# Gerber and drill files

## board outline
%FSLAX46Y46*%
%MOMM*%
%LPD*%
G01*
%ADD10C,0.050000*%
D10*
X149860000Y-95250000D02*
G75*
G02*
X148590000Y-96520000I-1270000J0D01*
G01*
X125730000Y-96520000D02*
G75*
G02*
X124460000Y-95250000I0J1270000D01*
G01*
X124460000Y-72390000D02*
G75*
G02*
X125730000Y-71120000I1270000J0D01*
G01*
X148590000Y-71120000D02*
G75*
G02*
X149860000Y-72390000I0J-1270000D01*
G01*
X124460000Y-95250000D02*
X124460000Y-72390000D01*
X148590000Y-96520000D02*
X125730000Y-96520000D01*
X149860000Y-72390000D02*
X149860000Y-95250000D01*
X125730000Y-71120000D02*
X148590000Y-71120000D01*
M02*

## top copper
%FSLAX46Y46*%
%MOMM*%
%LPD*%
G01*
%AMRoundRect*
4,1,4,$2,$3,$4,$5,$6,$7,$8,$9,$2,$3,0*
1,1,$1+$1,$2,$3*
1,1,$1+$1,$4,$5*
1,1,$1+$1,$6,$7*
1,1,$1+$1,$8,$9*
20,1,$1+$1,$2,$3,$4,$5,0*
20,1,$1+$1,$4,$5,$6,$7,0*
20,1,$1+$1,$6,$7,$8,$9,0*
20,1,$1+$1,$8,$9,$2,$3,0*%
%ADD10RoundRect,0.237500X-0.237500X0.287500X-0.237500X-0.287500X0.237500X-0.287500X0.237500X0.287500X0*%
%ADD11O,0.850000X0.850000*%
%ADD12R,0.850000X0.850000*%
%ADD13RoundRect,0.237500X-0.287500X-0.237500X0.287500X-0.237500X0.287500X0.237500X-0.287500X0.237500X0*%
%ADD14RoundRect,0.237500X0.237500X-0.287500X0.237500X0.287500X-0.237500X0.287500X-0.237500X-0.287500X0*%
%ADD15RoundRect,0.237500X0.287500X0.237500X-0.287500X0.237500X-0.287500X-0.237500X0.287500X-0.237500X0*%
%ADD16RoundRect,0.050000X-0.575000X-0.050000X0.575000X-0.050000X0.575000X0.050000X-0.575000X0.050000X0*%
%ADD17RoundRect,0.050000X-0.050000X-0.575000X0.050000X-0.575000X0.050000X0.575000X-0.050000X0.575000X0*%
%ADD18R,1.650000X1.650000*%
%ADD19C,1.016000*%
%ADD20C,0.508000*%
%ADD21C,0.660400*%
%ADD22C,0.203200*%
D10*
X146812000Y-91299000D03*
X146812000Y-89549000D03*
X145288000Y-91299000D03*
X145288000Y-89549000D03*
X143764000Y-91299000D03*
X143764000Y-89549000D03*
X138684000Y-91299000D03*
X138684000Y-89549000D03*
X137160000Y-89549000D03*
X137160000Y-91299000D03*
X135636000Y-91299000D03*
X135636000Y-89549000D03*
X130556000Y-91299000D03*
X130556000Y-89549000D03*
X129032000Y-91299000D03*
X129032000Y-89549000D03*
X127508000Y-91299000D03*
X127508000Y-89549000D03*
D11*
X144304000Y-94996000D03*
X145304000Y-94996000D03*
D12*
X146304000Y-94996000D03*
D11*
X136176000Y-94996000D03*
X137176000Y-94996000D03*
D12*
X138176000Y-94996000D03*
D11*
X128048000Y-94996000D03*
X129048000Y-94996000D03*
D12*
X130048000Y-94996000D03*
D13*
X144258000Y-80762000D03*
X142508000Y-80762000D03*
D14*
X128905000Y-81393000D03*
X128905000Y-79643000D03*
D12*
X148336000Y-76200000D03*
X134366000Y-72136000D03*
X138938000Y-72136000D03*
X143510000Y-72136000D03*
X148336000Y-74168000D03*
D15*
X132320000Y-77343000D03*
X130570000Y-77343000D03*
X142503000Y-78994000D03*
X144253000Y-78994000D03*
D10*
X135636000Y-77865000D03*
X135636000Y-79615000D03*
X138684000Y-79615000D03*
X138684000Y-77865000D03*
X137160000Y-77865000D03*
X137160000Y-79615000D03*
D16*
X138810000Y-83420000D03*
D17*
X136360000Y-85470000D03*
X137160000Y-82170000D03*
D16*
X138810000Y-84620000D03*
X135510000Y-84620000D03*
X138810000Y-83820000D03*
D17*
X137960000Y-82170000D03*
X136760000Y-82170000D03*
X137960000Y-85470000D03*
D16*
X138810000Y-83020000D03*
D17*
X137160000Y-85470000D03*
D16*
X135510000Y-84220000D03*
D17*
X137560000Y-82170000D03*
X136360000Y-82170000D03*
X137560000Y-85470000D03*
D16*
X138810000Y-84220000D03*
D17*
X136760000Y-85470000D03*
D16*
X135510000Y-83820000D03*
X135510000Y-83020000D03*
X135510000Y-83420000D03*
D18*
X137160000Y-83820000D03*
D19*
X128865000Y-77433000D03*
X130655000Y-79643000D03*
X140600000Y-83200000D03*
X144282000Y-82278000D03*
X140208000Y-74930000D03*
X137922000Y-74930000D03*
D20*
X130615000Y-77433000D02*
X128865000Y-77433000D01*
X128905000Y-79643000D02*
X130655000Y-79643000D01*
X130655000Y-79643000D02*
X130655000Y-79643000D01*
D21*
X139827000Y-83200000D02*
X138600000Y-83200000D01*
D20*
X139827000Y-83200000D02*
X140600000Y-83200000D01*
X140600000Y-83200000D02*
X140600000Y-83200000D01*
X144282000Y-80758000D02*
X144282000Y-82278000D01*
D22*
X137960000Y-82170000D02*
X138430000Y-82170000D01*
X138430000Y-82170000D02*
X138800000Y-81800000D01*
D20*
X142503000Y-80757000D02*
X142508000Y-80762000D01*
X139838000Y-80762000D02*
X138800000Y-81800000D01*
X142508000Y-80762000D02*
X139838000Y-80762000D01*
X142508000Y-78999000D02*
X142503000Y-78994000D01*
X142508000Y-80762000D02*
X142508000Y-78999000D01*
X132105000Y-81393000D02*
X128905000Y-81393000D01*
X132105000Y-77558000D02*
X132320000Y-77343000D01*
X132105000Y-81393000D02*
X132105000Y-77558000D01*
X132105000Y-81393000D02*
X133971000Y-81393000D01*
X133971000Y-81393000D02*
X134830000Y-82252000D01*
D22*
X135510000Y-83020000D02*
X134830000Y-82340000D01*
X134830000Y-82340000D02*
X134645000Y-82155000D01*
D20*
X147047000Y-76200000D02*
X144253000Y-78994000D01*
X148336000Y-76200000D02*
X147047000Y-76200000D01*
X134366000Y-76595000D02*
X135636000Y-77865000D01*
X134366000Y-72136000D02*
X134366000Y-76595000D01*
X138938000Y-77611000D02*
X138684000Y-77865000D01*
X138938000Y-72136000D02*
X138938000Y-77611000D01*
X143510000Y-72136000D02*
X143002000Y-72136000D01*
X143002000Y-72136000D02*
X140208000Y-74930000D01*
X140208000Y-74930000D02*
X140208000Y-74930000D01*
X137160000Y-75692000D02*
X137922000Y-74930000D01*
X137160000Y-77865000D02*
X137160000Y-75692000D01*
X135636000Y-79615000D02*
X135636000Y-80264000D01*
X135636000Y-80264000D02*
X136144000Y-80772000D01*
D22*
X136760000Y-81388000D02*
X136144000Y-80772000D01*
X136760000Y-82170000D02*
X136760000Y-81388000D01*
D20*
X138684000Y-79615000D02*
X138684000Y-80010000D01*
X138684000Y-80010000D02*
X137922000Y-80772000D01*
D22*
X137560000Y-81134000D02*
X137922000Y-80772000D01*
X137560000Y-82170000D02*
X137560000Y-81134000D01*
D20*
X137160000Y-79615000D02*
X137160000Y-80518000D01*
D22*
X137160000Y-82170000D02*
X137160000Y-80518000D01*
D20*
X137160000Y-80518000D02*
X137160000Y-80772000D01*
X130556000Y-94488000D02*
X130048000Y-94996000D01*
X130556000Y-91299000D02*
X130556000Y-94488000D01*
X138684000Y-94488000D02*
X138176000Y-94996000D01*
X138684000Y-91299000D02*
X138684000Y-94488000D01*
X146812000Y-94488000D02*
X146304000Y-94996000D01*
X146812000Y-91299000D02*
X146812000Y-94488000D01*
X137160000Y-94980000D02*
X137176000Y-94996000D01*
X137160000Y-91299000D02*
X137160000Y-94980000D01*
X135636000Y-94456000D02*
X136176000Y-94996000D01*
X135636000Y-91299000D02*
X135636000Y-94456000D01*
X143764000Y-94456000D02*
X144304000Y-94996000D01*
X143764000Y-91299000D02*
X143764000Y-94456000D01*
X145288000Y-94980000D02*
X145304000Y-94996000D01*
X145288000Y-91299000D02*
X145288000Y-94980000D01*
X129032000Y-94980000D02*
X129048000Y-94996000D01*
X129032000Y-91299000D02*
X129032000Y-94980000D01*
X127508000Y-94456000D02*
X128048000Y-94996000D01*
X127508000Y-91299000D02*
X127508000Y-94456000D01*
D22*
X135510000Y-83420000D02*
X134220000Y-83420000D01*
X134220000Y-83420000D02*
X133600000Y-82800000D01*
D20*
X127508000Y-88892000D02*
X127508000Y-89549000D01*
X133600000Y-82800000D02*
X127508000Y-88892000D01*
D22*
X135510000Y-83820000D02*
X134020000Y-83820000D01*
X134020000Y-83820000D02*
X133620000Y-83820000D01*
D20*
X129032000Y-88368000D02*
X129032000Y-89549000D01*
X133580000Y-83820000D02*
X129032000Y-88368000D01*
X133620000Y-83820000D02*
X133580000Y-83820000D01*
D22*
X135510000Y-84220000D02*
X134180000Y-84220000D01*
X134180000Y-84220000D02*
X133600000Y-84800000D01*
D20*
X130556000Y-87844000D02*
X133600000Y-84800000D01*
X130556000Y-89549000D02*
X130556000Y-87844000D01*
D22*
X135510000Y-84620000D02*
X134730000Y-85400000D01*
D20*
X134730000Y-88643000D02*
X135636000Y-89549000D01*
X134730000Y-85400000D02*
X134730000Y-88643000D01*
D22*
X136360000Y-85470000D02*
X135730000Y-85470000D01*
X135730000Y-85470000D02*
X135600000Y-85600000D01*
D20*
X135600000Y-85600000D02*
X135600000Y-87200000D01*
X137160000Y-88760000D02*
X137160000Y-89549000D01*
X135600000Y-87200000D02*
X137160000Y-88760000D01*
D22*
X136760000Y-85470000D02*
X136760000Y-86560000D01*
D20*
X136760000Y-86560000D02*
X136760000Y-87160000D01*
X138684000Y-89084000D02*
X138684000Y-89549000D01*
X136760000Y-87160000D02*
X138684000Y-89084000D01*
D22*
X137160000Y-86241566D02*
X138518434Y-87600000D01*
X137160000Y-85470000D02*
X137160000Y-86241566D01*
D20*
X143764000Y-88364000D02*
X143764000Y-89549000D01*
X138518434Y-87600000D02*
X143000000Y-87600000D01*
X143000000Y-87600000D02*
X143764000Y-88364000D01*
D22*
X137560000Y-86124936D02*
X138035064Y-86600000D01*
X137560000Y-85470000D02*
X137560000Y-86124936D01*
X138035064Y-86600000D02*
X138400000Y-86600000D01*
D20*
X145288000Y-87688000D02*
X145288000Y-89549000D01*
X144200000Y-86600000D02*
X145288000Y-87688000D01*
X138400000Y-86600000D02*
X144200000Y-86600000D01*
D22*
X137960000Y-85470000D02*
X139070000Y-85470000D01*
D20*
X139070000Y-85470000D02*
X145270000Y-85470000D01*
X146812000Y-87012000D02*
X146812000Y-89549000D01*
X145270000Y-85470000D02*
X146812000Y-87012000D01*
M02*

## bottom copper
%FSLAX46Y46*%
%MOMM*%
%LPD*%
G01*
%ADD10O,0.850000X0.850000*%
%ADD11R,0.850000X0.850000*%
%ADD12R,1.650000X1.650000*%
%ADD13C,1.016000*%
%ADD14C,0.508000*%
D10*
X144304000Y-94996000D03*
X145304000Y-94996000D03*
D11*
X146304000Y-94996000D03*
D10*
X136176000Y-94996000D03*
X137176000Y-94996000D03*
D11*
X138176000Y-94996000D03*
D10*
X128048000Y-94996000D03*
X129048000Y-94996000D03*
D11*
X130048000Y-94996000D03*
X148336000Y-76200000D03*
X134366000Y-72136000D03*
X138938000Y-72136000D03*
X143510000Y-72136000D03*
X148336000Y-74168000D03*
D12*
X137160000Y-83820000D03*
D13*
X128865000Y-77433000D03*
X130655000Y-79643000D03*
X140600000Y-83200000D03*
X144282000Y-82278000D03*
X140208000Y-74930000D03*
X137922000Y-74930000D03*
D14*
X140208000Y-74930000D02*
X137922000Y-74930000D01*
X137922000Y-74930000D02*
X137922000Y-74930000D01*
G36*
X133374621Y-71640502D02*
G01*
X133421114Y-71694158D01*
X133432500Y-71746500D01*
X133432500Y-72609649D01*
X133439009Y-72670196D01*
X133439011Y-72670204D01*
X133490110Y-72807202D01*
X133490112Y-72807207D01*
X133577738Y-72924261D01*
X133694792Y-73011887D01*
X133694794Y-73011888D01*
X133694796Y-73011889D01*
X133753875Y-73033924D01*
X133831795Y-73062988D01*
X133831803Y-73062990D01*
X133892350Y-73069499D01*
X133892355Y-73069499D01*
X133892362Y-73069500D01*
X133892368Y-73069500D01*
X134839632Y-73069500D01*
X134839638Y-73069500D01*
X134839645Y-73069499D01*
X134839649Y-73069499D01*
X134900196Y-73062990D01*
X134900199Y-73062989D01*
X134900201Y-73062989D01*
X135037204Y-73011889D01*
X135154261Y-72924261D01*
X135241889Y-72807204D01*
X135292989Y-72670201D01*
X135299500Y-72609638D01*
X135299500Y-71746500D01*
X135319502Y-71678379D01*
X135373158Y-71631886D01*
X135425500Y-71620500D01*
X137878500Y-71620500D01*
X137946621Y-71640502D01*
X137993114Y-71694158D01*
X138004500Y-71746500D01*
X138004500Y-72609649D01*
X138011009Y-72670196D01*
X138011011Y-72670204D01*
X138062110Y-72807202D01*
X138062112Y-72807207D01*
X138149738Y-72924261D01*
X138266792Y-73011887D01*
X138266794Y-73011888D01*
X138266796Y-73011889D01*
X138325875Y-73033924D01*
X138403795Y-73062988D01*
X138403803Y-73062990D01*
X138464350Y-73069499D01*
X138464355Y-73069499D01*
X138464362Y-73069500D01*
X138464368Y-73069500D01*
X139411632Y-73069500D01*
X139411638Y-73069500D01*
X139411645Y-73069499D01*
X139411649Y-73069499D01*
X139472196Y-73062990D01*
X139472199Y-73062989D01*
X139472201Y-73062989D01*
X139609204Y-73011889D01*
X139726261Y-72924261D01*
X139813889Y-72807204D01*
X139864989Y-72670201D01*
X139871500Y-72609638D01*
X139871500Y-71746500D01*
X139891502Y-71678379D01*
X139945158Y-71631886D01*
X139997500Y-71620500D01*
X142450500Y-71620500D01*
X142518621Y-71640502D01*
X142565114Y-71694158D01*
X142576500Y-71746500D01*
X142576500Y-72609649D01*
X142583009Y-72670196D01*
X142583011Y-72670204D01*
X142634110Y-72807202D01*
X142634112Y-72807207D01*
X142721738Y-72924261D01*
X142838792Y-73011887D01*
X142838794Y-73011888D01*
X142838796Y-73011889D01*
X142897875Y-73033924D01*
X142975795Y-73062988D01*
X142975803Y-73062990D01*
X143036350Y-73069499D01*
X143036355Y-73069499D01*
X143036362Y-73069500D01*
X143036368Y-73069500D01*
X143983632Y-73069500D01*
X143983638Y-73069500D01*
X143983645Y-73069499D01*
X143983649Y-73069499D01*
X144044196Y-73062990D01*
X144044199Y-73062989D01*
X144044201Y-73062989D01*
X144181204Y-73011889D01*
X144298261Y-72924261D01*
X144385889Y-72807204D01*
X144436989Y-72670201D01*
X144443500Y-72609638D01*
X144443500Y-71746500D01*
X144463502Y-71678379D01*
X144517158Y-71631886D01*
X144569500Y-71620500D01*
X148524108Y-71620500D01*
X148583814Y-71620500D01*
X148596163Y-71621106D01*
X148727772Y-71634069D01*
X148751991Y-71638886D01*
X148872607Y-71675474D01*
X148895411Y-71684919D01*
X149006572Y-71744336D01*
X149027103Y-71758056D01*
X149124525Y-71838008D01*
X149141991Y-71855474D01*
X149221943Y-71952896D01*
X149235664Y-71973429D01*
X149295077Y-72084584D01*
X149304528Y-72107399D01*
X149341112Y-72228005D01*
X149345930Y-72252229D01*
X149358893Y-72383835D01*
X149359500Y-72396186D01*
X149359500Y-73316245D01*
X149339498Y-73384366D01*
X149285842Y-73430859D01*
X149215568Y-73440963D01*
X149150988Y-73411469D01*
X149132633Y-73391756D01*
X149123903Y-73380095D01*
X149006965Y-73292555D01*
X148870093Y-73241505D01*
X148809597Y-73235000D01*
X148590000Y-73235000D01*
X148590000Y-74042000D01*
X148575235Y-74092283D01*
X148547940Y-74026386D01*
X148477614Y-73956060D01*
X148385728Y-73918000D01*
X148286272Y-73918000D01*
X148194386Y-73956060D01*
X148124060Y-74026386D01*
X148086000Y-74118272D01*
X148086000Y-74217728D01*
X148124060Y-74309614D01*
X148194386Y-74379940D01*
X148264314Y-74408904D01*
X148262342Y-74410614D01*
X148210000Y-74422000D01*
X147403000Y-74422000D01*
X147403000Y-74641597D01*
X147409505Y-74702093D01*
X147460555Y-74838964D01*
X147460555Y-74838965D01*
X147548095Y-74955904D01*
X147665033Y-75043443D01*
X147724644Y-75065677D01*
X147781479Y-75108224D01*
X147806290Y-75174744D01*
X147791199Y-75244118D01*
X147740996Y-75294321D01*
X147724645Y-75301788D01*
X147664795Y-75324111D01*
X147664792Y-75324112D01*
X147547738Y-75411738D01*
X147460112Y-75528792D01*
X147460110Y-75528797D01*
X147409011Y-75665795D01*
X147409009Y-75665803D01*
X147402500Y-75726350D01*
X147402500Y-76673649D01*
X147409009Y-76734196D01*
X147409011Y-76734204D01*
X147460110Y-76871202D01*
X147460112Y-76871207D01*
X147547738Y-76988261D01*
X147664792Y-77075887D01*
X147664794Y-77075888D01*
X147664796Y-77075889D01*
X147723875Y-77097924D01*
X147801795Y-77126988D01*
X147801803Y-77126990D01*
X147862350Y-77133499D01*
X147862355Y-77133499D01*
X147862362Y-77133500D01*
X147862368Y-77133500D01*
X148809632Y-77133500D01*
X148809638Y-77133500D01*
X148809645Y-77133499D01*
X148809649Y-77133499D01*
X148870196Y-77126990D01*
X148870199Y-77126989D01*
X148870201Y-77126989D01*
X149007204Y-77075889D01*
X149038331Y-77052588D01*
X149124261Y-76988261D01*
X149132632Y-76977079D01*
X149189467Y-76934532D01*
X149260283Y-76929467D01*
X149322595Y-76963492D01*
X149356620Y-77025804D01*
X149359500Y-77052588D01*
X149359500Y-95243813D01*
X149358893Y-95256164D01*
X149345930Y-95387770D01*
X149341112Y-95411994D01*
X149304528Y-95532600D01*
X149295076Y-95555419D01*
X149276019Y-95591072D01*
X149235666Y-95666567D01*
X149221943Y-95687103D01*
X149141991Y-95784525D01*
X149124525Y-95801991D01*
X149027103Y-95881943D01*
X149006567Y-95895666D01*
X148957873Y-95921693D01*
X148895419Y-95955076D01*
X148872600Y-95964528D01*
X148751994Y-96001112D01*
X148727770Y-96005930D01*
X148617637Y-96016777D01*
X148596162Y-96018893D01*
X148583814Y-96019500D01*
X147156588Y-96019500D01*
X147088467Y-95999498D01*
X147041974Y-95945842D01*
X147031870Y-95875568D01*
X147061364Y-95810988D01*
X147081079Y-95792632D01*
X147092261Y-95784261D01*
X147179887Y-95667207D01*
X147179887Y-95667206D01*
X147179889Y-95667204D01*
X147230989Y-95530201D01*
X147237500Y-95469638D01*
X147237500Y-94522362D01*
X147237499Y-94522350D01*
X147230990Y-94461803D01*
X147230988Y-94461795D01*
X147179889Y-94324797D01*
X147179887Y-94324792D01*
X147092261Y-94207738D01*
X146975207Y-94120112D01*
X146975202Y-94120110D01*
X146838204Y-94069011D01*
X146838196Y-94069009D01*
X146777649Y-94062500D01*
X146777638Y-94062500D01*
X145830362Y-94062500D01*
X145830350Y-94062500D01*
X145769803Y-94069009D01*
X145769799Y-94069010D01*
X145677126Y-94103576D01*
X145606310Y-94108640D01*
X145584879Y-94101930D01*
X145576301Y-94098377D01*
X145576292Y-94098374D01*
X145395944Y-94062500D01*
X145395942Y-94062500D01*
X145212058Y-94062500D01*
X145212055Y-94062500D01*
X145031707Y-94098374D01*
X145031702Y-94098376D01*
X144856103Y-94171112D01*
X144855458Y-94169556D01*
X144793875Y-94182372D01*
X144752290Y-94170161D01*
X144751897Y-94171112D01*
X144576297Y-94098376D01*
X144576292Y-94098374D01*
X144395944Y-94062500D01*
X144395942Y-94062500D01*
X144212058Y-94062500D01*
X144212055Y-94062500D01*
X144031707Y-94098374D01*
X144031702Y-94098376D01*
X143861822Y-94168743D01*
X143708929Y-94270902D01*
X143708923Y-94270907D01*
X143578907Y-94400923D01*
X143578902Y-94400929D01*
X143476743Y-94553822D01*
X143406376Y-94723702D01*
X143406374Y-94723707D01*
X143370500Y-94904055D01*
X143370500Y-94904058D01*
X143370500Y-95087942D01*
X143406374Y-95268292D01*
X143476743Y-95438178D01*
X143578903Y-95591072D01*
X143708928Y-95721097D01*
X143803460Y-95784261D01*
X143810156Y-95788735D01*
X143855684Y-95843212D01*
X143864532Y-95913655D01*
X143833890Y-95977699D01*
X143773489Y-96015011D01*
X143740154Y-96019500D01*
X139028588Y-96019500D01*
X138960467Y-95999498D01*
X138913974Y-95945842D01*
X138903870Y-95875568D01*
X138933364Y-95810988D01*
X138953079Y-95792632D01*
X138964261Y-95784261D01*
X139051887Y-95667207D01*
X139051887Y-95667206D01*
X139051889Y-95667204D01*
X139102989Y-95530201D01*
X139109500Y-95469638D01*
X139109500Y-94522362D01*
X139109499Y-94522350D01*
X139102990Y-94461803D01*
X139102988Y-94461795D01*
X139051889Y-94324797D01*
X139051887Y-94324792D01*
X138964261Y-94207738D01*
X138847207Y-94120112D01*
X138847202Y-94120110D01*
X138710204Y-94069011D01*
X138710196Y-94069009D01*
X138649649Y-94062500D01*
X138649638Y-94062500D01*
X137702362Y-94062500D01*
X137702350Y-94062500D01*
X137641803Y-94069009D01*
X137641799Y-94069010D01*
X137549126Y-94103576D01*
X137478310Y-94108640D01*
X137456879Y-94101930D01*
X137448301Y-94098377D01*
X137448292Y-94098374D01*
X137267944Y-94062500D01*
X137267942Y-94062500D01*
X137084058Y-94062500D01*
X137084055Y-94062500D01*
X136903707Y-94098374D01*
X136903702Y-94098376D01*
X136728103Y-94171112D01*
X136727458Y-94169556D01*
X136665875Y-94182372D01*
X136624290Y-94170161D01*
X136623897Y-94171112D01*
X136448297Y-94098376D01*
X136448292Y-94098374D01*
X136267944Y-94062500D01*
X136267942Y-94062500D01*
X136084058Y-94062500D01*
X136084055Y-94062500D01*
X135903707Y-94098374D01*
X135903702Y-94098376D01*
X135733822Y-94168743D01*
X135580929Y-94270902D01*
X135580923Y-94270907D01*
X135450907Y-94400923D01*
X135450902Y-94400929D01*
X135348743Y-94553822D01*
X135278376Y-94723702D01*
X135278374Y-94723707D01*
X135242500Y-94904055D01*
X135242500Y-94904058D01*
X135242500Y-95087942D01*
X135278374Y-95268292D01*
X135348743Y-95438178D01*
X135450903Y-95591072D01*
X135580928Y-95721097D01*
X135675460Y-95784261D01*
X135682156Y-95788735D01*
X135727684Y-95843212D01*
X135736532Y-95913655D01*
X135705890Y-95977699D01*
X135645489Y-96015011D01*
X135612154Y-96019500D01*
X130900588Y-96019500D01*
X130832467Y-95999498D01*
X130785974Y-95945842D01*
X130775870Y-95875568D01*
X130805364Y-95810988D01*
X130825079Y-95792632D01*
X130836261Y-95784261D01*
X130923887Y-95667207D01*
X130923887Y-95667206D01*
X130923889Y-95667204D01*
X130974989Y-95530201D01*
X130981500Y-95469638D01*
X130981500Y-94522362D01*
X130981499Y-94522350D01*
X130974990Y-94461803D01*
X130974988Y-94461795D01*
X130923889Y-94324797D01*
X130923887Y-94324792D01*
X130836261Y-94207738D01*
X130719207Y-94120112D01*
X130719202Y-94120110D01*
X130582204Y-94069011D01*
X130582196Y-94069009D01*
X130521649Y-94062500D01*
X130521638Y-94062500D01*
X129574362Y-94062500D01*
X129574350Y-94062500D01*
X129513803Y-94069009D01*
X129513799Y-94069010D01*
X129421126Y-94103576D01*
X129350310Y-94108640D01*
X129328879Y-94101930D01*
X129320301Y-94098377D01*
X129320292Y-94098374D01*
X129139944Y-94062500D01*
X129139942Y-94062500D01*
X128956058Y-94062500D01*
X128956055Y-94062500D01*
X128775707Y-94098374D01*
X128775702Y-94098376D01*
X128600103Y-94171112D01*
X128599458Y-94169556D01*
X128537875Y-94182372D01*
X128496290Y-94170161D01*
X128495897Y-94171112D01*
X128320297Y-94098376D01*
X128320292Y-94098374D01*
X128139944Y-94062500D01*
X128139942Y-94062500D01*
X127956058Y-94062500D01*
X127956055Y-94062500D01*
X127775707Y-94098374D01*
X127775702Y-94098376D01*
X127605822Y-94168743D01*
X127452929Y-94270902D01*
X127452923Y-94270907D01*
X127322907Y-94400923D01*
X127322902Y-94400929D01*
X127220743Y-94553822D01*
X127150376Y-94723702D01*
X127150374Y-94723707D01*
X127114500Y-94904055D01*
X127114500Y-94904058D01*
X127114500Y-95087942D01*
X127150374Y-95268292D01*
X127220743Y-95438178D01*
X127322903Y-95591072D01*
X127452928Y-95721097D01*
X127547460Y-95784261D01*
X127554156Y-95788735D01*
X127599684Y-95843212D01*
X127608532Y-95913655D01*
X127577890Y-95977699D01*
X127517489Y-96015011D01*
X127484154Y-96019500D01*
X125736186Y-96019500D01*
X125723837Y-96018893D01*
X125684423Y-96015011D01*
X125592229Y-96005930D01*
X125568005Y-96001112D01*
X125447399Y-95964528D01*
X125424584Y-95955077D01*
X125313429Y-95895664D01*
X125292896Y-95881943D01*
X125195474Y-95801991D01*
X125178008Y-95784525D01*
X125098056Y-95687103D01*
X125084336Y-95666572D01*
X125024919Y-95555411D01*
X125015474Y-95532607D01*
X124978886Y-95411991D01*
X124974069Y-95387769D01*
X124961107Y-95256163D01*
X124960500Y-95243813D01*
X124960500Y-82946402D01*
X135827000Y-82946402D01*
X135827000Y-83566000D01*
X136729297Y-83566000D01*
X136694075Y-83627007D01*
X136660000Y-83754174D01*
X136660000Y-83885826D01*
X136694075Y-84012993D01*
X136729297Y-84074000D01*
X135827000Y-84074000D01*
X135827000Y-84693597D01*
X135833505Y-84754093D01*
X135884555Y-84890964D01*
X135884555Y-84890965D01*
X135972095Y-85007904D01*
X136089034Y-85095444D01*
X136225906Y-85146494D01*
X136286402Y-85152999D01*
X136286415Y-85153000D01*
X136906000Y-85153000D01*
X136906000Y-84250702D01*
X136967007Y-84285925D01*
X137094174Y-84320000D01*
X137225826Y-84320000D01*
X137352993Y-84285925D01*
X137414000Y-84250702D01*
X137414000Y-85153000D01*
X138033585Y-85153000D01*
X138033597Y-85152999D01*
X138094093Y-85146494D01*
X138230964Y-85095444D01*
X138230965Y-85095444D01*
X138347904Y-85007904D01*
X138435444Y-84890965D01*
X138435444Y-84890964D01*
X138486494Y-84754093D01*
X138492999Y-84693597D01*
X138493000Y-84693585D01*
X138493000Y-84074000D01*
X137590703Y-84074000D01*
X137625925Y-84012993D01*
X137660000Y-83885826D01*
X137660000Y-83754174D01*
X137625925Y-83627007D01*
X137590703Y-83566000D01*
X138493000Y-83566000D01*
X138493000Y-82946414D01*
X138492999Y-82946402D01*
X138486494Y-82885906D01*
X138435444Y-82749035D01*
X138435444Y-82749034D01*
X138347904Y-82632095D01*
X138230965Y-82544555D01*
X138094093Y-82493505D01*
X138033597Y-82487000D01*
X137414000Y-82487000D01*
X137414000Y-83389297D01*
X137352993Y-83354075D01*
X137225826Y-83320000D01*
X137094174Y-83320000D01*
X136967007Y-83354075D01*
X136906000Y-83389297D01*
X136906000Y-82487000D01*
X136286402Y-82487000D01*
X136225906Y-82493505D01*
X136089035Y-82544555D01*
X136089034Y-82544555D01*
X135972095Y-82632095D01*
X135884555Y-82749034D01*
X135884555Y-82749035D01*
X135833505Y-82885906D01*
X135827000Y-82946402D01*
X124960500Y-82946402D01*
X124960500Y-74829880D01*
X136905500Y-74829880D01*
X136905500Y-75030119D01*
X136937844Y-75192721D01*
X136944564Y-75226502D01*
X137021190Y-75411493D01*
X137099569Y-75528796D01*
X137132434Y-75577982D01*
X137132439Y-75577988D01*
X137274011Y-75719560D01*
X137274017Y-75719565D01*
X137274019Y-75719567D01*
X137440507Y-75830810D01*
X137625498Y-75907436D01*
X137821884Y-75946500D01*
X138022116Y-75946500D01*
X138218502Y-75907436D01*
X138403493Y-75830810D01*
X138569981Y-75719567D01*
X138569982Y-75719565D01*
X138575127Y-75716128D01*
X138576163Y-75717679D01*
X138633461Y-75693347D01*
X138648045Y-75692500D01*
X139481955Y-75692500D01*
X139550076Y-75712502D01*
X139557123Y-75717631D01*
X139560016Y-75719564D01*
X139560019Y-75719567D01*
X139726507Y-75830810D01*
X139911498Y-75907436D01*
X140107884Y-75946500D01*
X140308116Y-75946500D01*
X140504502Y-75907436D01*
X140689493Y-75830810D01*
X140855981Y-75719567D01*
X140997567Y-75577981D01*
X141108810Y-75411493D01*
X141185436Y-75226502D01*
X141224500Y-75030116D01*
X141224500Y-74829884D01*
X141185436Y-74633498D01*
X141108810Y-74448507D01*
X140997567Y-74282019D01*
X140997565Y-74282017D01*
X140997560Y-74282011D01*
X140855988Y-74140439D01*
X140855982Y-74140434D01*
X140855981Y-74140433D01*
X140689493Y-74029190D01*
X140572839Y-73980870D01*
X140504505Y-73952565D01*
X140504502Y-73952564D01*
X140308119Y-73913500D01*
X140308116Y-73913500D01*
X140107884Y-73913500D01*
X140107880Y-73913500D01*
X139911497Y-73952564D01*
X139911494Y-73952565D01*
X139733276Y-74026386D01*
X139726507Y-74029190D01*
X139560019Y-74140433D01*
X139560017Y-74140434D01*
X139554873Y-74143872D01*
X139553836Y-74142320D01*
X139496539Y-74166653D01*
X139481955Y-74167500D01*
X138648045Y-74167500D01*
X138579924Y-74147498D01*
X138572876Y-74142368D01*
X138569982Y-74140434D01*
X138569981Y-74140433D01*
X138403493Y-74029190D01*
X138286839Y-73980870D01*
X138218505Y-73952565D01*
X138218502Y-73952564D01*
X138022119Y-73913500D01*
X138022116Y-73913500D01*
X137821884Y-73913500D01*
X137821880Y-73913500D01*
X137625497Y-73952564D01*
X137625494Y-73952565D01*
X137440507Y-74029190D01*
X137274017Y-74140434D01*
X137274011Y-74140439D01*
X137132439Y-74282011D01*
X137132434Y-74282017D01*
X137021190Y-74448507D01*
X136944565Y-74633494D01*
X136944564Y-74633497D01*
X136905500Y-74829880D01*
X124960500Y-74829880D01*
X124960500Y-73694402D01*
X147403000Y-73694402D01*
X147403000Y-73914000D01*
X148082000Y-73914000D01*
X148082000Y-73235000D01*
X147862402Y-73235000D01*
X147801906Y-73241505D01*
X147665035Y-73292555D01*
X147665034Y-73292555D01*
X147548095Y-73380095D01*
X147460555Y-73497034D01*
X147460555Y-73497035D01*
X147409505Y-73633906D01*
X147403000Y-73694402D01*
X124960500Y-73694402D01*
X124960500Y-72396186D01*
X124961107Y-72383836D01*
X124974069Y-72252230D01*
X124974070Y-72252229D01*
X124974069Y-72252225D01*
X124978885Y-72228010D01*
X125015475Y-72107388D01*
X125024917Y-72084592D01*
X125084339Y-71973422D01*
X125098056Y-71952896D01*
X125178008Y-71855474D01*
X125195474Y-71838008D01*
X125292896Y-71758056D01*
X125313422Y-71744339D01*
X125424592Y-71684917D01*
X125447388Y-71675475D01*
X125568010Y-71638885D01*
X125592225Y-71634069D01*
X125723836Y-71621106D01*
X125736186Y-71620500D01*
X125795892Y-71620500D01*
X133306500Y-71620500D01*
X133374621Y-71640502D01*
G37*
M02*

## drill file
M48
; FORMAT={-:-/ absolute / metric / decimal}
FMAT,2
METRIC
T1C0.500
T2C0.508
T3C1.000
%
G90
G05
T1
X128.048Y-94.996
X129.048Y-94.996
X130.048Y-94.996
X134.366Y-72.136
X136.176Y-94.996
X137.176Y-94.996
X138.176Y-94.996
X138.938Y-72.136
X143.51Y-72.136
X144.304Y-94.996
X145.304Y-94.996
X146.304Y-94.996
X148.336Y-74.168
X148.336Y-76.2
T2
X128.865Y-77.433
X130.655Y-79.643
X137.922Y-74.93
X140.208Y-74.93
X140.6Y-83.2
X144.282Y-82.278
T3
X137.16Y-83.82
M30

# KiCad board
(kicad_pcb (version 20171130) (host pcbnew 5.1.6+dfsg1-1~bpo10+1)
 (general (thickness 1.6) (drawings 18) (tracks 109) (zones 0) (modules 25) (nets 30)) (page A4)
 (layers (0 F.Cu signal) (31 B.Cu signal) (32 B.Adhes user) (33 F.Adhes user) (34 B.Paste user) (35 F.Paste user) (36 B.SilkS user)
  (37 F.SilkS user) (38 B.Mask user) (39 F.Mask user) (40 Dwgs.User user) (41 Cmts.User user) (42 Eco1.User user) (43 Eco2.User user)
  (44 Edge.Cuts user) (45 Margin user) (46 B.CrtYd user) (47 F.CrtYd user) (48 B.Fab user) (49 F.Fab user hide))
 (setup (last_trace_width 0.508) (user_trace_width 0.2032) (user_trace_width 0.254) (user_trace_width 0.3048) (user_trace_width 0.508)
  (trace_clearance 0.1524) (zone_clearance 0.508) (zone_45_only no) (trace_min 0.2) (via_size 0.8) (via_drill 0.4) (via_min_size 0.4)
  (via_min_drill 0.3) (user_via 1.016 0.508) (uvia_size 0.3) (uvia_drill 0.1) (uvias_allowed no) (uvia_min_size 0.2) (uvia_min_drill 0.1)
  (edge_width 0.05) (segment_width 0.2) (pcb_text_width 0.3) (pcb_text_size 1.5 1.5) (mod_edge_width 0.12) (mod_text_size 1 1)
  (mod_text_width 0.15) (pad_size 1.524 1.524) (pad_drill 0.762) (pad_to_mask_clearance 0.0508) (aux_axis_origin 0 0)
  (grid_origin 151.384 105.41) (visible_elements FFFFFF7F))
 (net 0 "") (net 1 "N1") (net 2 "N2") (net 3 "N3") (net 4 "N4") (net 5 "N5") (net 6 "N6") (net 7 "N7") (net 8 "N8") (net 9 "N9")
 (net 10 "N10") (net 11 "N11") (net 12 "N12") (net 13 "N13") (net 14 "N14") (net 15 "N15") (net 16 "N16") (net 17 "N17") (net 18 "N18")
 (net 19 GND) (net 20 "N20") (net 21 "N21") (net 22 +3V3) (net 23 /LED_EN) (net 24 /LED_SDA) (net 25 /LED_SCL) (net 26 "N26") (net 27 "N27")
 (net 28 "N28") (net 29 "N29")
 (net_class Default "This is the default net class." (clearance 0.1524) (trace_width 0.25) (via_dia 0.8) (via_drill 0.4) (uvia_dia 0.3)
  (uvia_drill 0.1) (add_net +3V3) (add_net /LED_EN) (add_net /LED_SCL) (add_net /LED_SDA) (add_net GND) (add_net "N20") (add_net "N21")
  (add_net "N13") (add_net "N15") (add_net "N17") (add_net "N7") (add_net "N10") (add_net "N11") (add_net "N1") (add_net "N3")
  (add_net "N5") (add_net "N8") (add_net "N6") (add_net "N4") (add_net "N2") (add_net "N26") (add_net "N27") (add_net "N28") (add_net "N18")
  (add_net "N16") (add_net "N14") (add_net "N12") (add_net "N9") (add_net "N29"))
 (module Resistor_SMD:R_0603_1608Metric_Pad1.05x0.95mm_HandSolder (layer F.Cu) (at 146.812 90.424 270)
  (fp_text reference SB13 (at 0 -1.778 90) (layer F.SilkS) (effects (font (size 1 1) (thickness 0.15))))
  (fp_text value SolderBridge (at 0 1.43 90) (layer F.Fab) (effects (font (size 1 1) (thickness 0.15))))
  (pad 2 smd roundrect (at 0.875 0 270) (size 1.05 0.95) (layers F.Cu F.Paste F.Mask) (roundrect_rratio 0.25) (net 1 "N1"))
  (pad 1 smd roundrect (at -0.875 0 270) (size 1.05 0.95) (layers F.Cu F.Paste F.Mask) (roundrect_rratio 0.25) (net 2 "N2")))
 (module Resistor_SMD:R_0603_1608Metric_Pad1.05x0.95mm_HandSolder (layer F.Cu) (at 145.288 90.424 270)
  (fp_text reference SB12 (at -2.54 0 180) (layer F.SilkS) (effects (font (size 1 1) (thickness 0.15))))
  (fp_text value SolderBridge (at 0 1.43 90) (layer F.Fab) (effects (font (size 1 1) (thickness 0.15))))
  (pad 2 smd roundrect (at 0.875 0 270) (size 1.05 0.95) (layers F.Cu F.Paste F.Mask) (roundrect_rratio 0.25) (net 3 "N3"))
  (pad 1 smd roundrect (at -0.875 0 270) (size 1.05 0.95) (layers F.Cu F.Paste F.Mask) (roundrect_rratio 0.25) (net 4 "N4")))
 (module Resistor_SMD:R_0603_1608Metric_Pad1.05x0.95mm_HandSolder (layer F.Cu) (at 143.764 90.424 270)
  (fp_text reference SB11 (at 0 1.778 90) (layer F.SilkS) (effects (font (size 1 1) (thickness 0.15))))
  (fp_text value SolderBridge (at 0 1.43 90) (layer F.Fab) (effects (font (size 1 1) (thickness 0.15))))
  (pad 2 smd roundrect (at 0.875 0 270) (size 1.05 0.95) (layers F.Cu F.Paste F.Mask) (roundrect_rratio 0.25) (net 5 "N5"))
  (pad 1 smd roundrect (at -0.875 0 270) (size 1.05 0.95) (layers F.Cu F.Paste F.Mask) (roundrect_rratio 0.25) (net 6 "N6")))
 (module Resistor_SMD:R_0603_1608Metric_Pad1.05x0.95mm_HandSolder (layer F.Cu) (at 138.684 90.424 270)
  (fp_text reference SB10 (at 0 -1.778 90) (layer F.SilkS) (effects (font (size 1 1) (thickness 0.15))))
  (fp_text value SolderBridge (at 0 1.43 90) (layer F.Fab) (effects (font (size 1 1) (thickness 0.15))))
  (pad 2 smd roundrect (at 0.875 0 270) (size 1.05 0.95) (layers F.Cu F.Paste F.Mask) (roundrect_rratio 0.25) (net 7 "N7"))
  (pad 1 smd roundrect (at -0.875 0 270) (size 1.05 0.95) (layers F.Cu F.Paste F.Mask) (roundrect_rratio 0.25) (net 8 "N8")))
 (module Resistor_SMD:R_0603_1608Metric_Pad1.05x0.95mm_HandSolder (layer F.Cu) (at 137.16 90.424 270)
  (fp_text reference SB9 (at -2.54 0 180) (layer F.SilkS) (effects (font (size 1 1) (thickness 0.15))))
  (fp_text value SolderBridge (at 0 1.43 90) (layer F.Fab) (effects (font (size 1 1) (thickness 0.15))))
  (pad 1 smd roundrect (at -0.875 0 270) (size 1.05 0.95) (layers F.Cu F.Paste F.Mask) (roundrect_rratio 0.25) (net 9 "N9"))
  (pad 2 smd roundrect (at 0.875 0 270) (size 1.05 0.95) (layers F.Cu F.Paste F.Mask) (roundrect_rratio 0.25) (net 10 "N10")))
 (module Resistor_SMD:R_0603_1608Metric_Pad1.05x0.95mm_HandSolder (layer F.Cu) (at 135.636 90.424 270)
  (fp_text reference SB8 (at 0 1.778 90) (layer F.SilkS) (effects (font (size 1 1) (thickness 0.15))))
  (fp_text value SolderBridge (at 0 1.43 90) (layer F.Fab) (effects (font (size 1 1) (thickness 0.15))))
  (pad 2 smd roundrect (at 0.875 0 270) (size 1.05 0.95) (layers F.Cu F.Paste F.Mask) (roundrect_rratio 0.25) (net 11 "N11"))
  (pad 1 smd roundrect (at -0.875 0 270) (size 1.05 0.95) (layers F.Cu F.Paste F.Mask) (roundrect_rratio 0.25) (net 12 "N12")))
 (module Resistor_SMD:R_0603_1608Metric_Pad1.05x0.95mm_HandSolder (layer F.Cu) (at 130.556 90.424 270)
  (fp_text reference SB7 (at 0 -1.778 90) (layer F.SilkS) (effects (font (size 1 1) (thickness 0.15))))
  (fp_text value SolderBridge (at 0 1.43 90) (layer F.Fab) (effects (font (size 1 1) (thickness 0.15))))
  (pad 2 smd roundrect (at 0.875 0 270) (size 1.05 0.95) (layers F.Cu F.Paste F.Mask) (roundrect_rratio 0.25) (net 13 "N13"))
  (pad 1 smd roundrect (at -0.875 0 270) (size 1.05 0.95) (layers F.Cu F.Paste F.Mask) (roundrect_rratio 0.25) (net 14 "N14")))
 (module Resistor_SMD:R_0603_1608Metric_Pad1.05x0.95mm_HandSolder (layer F.Cu) (at 129.032 90.424 270)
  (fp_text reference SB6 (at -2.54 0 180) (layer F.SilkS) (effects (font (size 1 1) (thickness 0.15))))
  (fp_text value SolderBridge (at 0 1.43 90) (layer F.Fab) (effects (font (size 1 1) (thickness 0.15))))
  (pad 2 smd roundrect (at 0.875 0 270) (size 1.05 0.95) (layers F.Cu F.Paste F.Mask) (roundrect_rratio 0.25) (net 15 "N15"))
  (pad 1 smd roundrect (at -0.875 0 270) (size 1.05 0.95) (layers F.Cu F.Paste F.Mask) (roundrect_rratio 0.25) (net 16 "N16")))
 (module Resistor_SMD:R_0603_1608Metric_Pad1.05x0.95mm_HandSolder (layer F.Cu) (at 127.508 90.424 270)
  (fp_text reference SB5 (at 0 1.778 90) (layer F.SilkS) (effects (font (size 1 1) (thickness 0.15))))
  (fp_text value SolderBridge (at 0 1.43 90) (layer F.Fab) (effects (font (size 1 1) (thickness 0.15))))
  (pad 2 smd roundrect (at 0.875 0 270) (size 1.05 0.95) (layers F.Cu F.Paste F.Mask) (roundrect_rratio 0.25) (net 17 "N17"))
  (pad 1 smd roundrect (at -0.875 0 270) (size 1.05 0.95) (layers F.Cu F.Paste F.Mask) (roundrect_rratio 0.25) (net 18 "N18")))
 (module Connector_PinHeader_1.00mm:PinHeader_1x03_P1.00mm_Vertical (layer F.Cu) (at 146.304 94.996 270)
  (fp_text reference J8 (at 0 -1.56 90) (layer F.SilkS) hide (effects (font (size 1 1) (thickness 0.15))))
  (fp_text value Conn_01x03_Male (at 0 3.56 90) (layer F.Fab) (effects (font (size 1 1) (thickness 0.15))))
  (pad 3 thru_hole oval (at 0 2 270) (size 0.85 0.85) (drill 0.5) (layers *.Cu *.Mask) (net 5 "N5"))
  (pad 2 thru_hole oval (at 0 1 270) (size 0.85 0.85) (drill 0.5) (layers *.Cu *.Mask) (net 3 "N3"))
  (pad 1 thru_hole rect (at 0 0 270) (size 0.85 0.85) (drill 0.5) (layers *.Cu *.Mask) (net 1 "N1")))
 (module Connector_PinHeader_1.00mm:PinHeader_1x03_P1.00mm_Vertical (layer F.Cu) (at 138.176 94.996 270)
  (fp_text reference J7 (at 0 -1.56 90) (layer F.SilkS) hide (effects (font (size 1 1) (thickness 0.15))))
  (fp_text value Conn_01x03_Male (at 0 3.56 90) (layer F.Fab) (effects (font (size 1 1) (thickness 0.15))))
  (pad 3 thru_hole oval (at 0 2 270) (size 0.85 0.85) (drill 0.5) (layers *.Cu *.Mask) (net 11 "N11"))
  (pad 2 thru_hole oval (at 0 1 270) (size 0.85 0.85) (drill 0.5) (layers *.Cu *.Mask) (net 10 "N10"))
  (pad 1 thru_hole rect (at 0 0 270) (size 0.85 0.85) (drill 0.5) (layers *.Cu *.Mask) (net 7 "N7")))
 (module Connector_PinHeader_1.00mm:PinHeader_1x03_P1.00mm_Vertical (layer F.Cu) (at 130.048 94.996 270)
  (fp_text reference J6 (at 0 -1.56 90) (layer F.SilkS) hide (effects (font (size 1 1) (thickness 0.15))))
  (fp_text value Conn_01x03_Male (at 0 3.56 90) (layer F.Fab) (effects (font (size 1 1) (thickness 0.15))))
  (pad 3 thru_hole oval (at 0 2 270) (size 0.85 0.85) (drill 0.5) (layers *.Cu *.Mask) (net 17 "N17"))
  (pad 2 thru_hole oval (at 0 1 270) (size 0.85 0.85) (drill 0.5) (layers *.Cu *.Mask) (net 15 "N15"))
  (pad 1 thru_hole rect (at 0 0 270) (size 0.85 0.85) (drill 0.5) (layers *.Cu *.Mask) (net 13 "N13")))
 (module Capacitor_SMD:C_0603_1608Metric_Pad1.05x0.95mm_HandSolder (layer F.Cu) (at 143.383 80.762)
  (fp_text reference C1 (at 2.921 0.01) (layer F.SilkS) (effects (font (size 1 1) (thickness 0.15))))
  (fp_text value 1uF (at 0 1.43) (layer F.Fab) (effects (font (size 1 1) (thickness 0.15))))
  (pad 2 smd roundrect (at 0.875 0) (size 1.05 0.95) (layers F.Cu F.Paste F.Mask) (roundrect_rratio 0.25) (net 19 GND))
  (pad 1 smd roundrect (at -0.875 0) (size 1.05 0.95) (layers F.Cu F.Paste F.Mask) (roundrect_rratio 0.25) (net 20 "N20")))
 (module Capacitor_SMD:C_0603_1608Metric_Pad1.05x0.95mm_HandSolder (layer F.Cu) (at 128.905 80.518 90)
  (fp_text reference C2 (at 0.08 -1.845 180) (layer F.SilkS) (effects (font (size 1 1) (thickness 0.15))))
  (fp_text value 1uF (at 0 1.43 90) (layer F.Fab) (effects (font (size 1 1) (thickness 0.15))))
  (pad 1 smd roundrect (at -0.875 0 90) (size 1.05 0.95) (layers F.Cu F.Paste F.Mask) (roundrect_rratio 0.25) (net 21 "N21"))
  (pad 2 smd roundrect (at 0.875 0 90) (size 1.05 0.95) (layers F.Cu F.Paste F.Mask) (roundrect_rratio 0.25) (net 19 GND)))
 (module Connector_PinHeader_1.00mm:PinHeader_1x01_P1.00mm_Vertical (layer F.Cu) (at 148.336 76.2)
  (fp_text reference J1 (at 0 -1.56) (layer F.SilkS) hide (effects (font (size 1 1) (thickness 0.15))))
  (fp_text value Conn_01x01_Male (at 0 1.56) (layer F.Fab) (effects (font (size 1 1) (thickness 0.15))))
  (pad 1 thru_hole rect (at 0 0) (size 0.85 0.85) (drill 0.5) (layers *.Cu *.Mask) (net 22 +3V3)))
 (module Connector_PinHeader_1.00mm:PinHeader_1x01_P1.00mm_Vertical (layer F.Cu) (at 134.366 72.136)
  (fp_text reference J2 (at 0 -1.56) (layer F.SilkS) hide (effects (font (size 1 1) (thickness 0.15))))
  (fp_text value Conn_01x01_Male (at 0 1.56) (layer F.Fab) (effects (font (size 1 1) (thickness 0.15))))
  (pad 1 thru_hole rect (at 0 0) (size 0.85 0.85) (drill 0.5) (layers *.Cu *.Mask) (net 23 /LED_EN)))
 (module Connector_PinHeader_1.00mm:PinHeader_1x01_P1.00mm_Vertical (layer F.Cu) (at 138.938 72.136)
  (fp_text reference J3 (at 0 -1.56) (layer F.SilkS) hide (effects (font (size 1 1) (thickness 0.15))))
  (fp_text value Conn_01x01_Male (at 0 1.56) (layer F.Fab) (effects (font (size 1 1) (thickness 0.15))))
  (pad 1 thru_hole rect (at 0 0) (size 0.85 0.85) (drill 0.5) (layers *.Cu *.Mask) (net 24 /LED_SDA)))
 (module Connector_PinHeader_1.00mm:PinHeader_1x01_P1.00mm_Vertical (layer F.Cu) (at 143.51 72.136)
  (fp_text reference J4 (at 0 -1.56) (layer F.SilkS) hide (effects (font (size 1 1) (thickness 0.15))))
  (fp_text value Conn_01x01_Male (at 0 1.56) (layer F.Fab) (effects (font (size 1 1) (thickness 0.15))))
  (pad 1 thru_hole rect (at 0 0) (size 0.85 0.85) (drill 0.5) (layers *.Cu *.Mask) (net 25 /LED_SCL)))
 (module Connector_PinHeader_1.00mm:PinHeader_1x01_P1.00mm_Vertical (layer F.Cu) (at 148.336 74.168)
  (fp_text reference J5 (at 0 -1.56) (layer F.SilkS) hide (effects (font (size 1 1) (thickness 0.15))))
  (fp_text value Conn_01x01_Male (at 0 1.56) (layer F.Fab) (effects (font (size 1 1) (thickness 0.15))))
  (pad 1 thru_hole rect (at 0 0) (size 0.85 0.85) (drill 0.5) (layers *.Cu *.Mask) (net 19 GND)))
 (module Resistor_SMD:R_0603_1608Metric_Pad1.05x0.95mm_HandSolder (layer F.Cu) (at 131.445 77.343 180)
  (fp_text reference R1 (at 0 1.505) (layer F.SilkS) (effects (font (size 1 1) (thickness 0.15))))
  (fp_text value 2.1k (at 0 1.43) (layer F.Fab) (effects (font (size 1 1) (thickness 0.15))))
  (pad 1 smd roundrect (at -0.875 0 180) (size 1.05 0.95) (layers F.Cu F.Paste F.Mask) (roundrect_rratio 0.25) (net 21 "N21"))
  (pad 2 smd roundrect (at 0.875 0 180) (size 1.05 0.95) (layers F.Cu F.Paste F.Mask) (roundrect_rratio 0.25) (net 19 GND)))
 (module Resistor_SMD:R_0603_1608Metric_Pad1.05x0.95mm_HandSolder (layer F.Cu) (at 143.378 78.994 180)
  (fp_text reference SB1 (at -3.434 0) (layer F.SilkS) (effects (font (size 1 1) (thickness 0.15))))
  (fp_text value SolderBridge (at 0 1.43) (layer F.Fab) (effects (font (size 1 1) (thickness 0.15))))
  (pad 2 smd roundrect (at 0.875 0 180) (size 1.05 0.95) (layers F.Cu F.Paste F.Mask) (roundrect_rratio 0.25) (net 20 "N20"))
  (pad 1 smd roundrect (at -0.875 0 180) (size 1.05 0.95) (layers F.Cu F.Paste F.Mask) (roundrect_rratio 0.25) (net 22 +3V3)))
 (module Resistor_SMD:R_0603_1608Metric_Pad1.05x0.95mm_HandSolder (layer F.Cu) (at 135.636 78.74 270)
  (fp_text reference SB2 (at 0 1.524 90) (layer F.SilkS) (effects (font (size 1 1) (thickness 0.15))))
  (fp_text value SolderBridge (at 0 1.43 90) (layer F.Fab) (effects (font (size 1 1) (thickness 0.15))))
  (pad 1 smd roundrect (at -0.875 0 270) (size 1.05 0.95) (layers F.Cu F.Paste F.Mask) (roundrect_rratio 0.25) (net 23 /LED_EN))
  (pad 2 smd roundrect (at 0.875 0 270) (size 1.05 0.95) (layers F.Cu F.Paste F.Mask) (roundrect_rratio 0.25) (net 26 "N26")))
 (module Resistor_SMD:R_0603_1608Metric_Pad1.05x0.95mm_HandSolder (layer F.Cu) (at 138.684 78.74 270)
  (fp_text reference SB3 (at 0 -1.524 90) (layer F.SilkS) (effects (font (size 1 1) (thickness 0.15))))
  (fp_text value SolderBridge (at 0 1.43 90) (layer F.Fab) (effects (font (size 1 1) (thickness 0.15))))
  (pad 2 smd roundrect (at 0.875 0 270) (size 1.05 0.95) (layers F.Cu F.Paste F.Mask) (roundrect_rratio 0.25) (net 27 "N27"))
  (pad 1 smd roundrect (at -0.875 0 270) (size 1.05 0.95) (layers F.Cu F.Paste F.Mask) (roundrect_rratio 0.25) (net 24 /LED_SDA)))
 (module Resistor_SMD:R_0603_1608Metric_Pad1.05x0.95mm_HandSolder (layer F.Cu) (at 137.16 78.74 270)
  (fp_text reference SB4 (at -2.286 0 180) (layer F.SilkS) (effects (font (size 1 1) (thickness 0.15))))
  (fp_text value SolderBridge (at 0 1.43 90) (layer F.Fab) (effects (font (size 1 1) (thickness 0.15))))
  (pad 1 smd roundrect (at -0.875 0 270) (size 1.05 0.95) (layers F.Cu F.Paste F.Mask) (roundrect_rratio 0.25) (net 25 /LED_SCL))
  (pad 2 smd roundrect (at 0.875 0 270) (size 1.05 0.95) (layers F.Cu F.Paste F.Mask) (roundrect_rratio 0.25) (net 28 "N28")))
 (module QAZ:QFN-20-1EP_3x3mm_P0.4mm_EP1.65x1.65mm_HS (layer F.Cu) (at 137.16 83.82)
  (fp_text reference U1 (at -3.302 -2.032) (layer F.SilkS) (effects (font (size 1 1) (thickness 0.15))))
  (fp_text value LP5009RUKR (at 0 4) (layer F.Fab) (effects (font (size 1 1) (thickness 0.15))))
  (pad 14 smd roundrect (at 1.65 -0.4) (size 1.25 0.2) (layers F.Cu F.Paste F.Mask) (roundrect_rratio 0.25) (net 19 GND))
  (pad 6 smd roundrect (at -0.8 1.65) (size 0.2 1.25) (layers F.Cu F.Paste F.Mask) (roundrect_rratio 0.25) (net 9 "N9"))
  (pad 18 smd roundrect (at 0 -1.65) (size 0.2 1.25) (layers F.Cu F.Paste F.Mask) (roundrect_rratio 0.25) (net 28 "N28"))
  (pad 11 smd roundrect (at 1.65 0.8) (size 1.25 0.2) (layers F.Cu F.Paste F.Mask) (roundrect_rratio 0.25))
  (pad 5 smd roundrect (at -1.65 0.8) (size 1.25 0.2) (layers F.Cu F.Paste F.Mask) (roundrect_rratio 0.25) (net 12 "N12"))
  (pad 13 smd roundrect (at 1.65 0) (size 1.25 0.2) (layers F.Cu F.Paste F.Mask) (roundrect_rratio 0.25))
  (pad 16 smd roundrect (at 0.8 -1.65) (size 0.2 1.25) (layers F.Cu F.Paste F.Mask) (roundrect_rratio 0.25) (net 20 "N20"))
  (pad 19 smd roundrect (at -0.4 -1.65) (size 0.2 1.25) (layers F.Cu F.Paste F.Mask) (roundrect_rratio 0.25) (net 26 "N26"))
  (pad 10 smd roundrect (at 0.8 1.65) (size 0.2 1.25) (layers F.Cu F.Paste F.Mask) (roundrect_rratio 0.25) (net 2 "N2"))
  (pad 15 smd roundrect (at 1.65 -0.8) (size 1.25 0.2) (layers F.Cu F.Paste F.Mask) (roundrect_rratio 0.25) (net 19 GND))
  (pad 8 smd roundrect (at 0 1.65) (size 0.2 1.25) (layers F.Cu F.Paste F.Mask) (roundrect_rratio 0.25) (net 6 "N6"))
  (pad 4 smd roundrect (at -1.65 0.4) (size 1.25 0.2) (layers F.Cu F.Paste F.Mask) (roundrect_rratio 0.25) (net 14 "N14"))
  (pad 17 smd roundrect (at 0.4 -1.65) (size 0.2 1.25) (layers F.Cu F.Paste F.Mask) (roundrect_rratio 0.25) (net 27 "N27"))
  (pad 20 smd roundrect (at -0.8 -1.65) (size 0.2 1.25) (layers F.Cu F.Paste F.Mask) (roundrect_rratio 0.25) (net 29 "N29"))
  (pad 9 smd roundrect (at 0.4 1.65) (size 0.2 1.25) (layers F.Cu F.Paste F.Mask) (roundrect_rratio 0.25) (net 4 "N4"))
  (pad 12 smd roundrect (at 1.65 0.4) (size 1.25 0.2) (layers F.Cu F.Paste F.Mask) (roundrect_rratio 0.25))
  (pad 7 smd roundrect (at -0.4 1.65) (size 0.2 1.25) (layers F.Cu F.Paste F.Mask) (roundrect_rratio 0.25) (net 8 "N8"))
  (pad 3 smd roundrect (at -1.65 0) (size 1.25 0.2) (layers F.Cu F.Paste F.Mask) (roundrect_rratio 0.25) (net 16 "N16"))
  (pad 1 smd roundrect (at -1.65 -0.8) (size 1.25 0.2) (layers F.Cu F.Paste F.Mask) (roundrect_rratio 0.25) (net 21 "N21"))
  (pad 2 smd roundrect (at -1.65 -0.4) (size 1.25 0.2) (layers F.Cu F.Paste F.Mask) (roundrect_rratio 0.25) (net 18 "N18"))
  (pad 21 thru_hole rect (at 0 0) (size 1.65 1.65) (drill 1) (layers *.Cu *.Mask) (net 19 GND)))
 (gr_arc (start 148.59 95.25) (end 148.59 96.52) (angle -90) (layer Edge.Cuts) (width 0.05))
 (gr_arc (start 125.73 95.25) (end 124.46 95.25) (angle -90) (layer Edge.Cuts) (width 0.05))
 (gr_arc (start 125.73 72.39) (end 125.73 71.12) (angle -90) (layer Edge.Cuts) (width 0.05))
 (gr_arc (start 148.59 72.39) (end 149.86 72.39) (angle -90) (layer Edge.Cuts) (width 0.05))
 (gr_line (start 124.46 95.25) (end 124.46 72.39) (layer Edge.Cuts) (width 0.05))
 (gr_line (start 148.59 96.52) (end 125.73 96.52) (layer Edge.Cuts) (width 0.05))
 (gr_line (start 149.86 72.39) (end 149.86 95.25) (layer Edge.Cuts) (width 0.05))
 (gr_line (start 125.73 71.12) (end 148.59 71.12) (layer Edge.Cuts) (width 0.05))
 (via (at 128.865 77.433) (size 1.016) (drill 0.508) (layers F.Cu B.Cu) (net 19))
 (segment (start 130.615 77.433) (end 128.865 77.433) (width 0.508) (layer F.Cu) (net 19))
 (segment (start 128.905 79.643) (end 130.655 79.643) (width 0.508) (layer F.Cu) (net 19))
 (segment (start 130.655 79.643) (end 130.655 79.643) (width 0.508) (layer F.Cu) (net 19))
 (via (at 130.655 79.643) (size 1.016) (drill 0.508) (layers F.Cu B.Cu) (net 19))
 (segment (start 139.827 83.2) (end 138.6 83.2) (width 0.6604) (layer F.Cu) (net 19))
 (segment (start 139.827 83.2) (end 140.6 83.2) (width 0.508) (layer F.Cu) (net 19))
 (segment (start 140.6 83.2) (end 140.6 83.2) (width 0.508) (layer F.Cu) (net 19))
 (via (at 140.6 83.2) (size 1.016) (drill 0.508) (layers F.Cu B.Cu) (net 19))
 (segment (start 144.282 80.758) (end 144.282 82.278) (width 0.508) (layer F.Cu) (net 19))
 (via (at 144.282 82.278) (size 1.016) (drill 0.508) (layers F.Cu B.Cu) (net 19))
 (segment (start 137.96 82.17) (end 138.43 82.17) (width 0.2032) (layer F.Cu) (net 20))
 (segment (start 138.43 82.17) (end 138.8 81.8) (width 0.2032) (layer F.Cu) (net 20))
 (segment (start 142.503 80.757) (end 142.508 80.762) (width 0.508) (layer F.Cu) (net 20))
 (segment (start 139.838 80.762) (end 138.8 81.8) (width 0.508) (layer F.Cu) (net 20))
 (segment (start 142.508 80.762) (end 139.838 80.762) (width 0.508) (layer F.Cu) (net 20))
 (segment (start 142.508 78.999) (end 142.503 78.994) (width 0.508) (layer F.Cu) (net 20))
 (segment (start 142.508 80.762) (end 142.508 78.999) (width 0.508) (layer F.Cu) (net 20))
 (segment (start 132.105 81.393) (end 128.905 81.393) (width 0.508) (layer F.Cu) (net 21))
 (segment (start 132.105 77.558) (end 132.32 77.343) (width 0.508) (layer F.Cu) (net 21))
 (segment (start 132.105 81.393) (end 132.105 77.558) (width 0.508) (layer F.Cu) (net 21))
 (segment (start 132.105 81.393) (end 133.971 81.393) (width 0.508) (layer F.Cu) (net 21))
 (segment (start 133.971 81.393) (end 134.83 82.252) (width 0.508) (layer F.Cu) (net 21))
 (segment (start 135.51 83.02) (end 134.83 82.34) (width 0.2032) (layer F.Cu) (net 21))
 (segment (start 134.83 82.34) (end 134.645 82.155) (width 0.2032) (layer F.Cu) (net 21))
 (segment (start 147.047 76.2) (end 144.253 78.994) (width 0.508) (layer F.Cu) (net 22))
 (segment (start 148.336 76.2) (end 147.047 76.2) (width 0.508) (layer F.Cu) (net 22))
 (segment (start 134.366 76.595) (end 135.636 77.865) (width 0.508) (layer F.Cu) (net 23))
 (segment (start 134.366 72.136) (end 134.366 76.595) (width 0.508) (layer F.Cu) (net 23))
 (segment (start 138.938 77.611) (end 138.684 77.865) (width 0.508) (layer F.Cu) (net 24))
 (segment (start 138.938 72.136) (end 138.938 77.611) (width 0.508) (layer F.Cu) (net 24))
 (segment (start 143.51 72.136) (end 143.002 72.136) (width 0.508) (layer F.Cu) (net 25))
 (segment (start 143.002 72.136) (end 140.208 74.93) (width 0.508) (layer F.Cu) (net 25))
 (segment (start 140.208 74.93) (end 140.208 74.93) (width 0.508) (layer F.Cu) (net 25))
 (via (at 140.208 74.93) (size 1.016) (drill 0.508) (layers F.Cu B.Cu) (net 25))
 (segment (start 140.208 74.93) (end 137.922 74.93) (width 0.508) (layer B.Cu) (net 25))
 (segment (start 137.922 74.93) (end 137.922 74.93) (width 0.508) (layer B.Cu) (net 25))
 (via (at 137.922 74.93) (size 1.016) (drill 0.508) (layers F.Cu B.Cu) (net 25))
 (segment (start 137.16 75.692) (end 137.922 74.93) (width 0.508) (layer F.Cu) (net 25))
 (segment (start 137.16 77.865) (end 137.16 75.692) (width 0.508) (layer F.Cu) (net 25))
 (segment (start 135.636 79.615) (end 135.636 80.264) (width 0.508) (layer F.Cu) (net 26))
 (segment (start 135.636 80.264) (end 136.144 80.772) (width 0.508) (layer F.Cu) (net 26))
 (segment (start 136.76 81.388) (end 136.144 80.772) (width 0.2032) (layer F.Cu) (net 26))
 (segment (start 136.76 82.17) (end 136.76 81.388) (width 0.2032) (layer F.Cu) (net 26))
 (segment (start 138.684 79.615) (end 138.684 80.01) (width 0.508) (layer F.Cu) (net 27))
 (segment (start 138.684 80.01) (end 137.922 80.772) (width 0.508) (layer F.Cu) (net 27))
 (segment (start 137.56 81.134) (end 137.922 80.772) (width 0.2032) (layer F.Cu) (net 27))
 (segment (start 137.56 82.17) (end 137.56 81.134) (width 0.2032) (layer F.Cu) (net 27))
 (segment (start 137.16 79.615) (end 137.16 80.518) (width 0.508) (layer F.Cu) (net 28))
 (segment (start 137.16 82.17) (end 137.16 80.518) (width 0.2032) (layer F.Cu) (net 28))
 (segment (start 137.16 80.518) (end 137.16 80.772) (width 0.508) (layer F.Cu) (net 28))
 (segment (start 130.556 94.488) (end 130.048 94.996) (width 0.508) (layer F.Cu) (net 13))
 (segment (start 130.556 91.299) (end 130.556 94.488) (width 0.508) (layer F.Cu) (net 13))
 (segment (start 138.684 94.488) (end 138.176 94.996) (width 0.508) (layer F.Cu) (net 7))
 (segment (start 138.684 91.299) (end 138.684 94.488) (width 0.508) (layer F.Cu) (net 7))
 (segment (start 146.812 94.488) (end 146.304 94.996) (width 0.508) (layer F.Cu) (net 1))
 (segment (start 146.812 91.299) (end 146.812 94.488) (width 0.508) (layer F.Cu) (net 1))
 (segment (start 137.16 94.98) (end 137.176 94.996) (width 0.508) (layer F.Cu) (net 10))
 (segment (start 137.16 91.299) (end 137.16 94.98) (width 0.508) (layer F.Cu) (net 10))
 (segment (start 135.636 94.456) (end 136.176 94.996) (width 0.508) (layer F.Cu) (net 11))
 (segment (start 135.636 91.299) (end 135.636 94.456) (width 0.508) (layer F.Cu) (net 11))
 (segment (start 143.764 94.456) (end 144.304 94.996) (width 0.508) (layer F.Cu) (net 5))
 (segment (start 143.764 91.299) (end 143.764 94.456) (width 0.508) (layer F.Cu) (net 5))
 (segment (start 145.288 94.98) (end 145.304 94.996) (width 0.508) (layer F.Cu) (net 3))
 (segment (start 145.288 91.299) (end 145.288 94.98) (width 0.508) (layer F.Cu) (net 3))
 (segment (start 129.032 94.98) (end 129.048 94.996) (width 0.508) (layer F.Cu) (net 15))
 (segment (start 129.032 91.299) (end 129.032 94.98) (width 0.508) (layer F.Cu) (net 15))
 (segment (start 127.508 94.456) (end 128.048 94.996) (width 0.508) (layer F.Cu) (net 17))
 (segment (start 127.508 91.299) (end 127.508 94.456) (width 0.508) (layer F.Cu) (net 17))
 (segment (start 135.51 83.42) (end 134.22 83.42) (width 0.2032) (layer F.Cu) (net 18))
 (segment (start 134.22 83.42) (end 133.6 82.8) (width 0.2032) (layer F.Cu) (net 18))
 (segment (start 127.508 88.892) (end 127.508 89.549) (width 0.508) (layer F.Cu) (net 18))
 (segment (start 133.6 82.8) (end 127.508 88.892) (width 0.508) (layer F.Cu) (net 18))
 (segment (start 135.51 83.82) (end 134.02 83.82) (width 0.2032) (layer F.Cu) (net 16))
 (segment (start 134.02 83.82) (end 133.62 83.82) (width 0.2032) (layer F.Cu) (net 16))
 (segment (start 129.032 88.368) (end 129.032 89.549) (width 0.508) (layer F.Cu) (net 16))
 (segment (start 133.58 83.82) (end 129.032 88.368) (width 0.508) (layer F.Cu) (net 16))
 (segment (start 133.62 83.82) (end 133.58 83.82) (width 0.508) (layer F.Cu) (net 16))
 (segment (start 135.51 84.22) (end 134.18 84.22) (width 0.2032) (layer F.Cu) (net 14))
 (segment (start 134.18 84.22) (end 133.6 84.8) (width 0.2032) (layer F.Cu) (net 14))
 (segment (start 130.556 87.844) (end 133.6 84.8) (width 0.508) (layer F.Cu) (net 14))
 (segment (start 130.556 89.549) (end 130.556 87.844) (width 0.508) (layer F.Cu) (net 14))
 (segment (start 135.51 84.62) (end 134.73 85.4) (width 0.2032) (layer F.Cu) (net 12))
 (segment (start 134.73 88.643) (end 135.636 89.549) (width 0.508) (layer F.Cu) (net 12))
 (segment (start 134.73 85.4) (end 134.73 88.643) (width 0.508) (layer F.Cu) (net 12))
 (segment (start 136.36 85.47) (end 135.73 85.47) (width 0.2032) (layer F.Cu) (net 9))
 (segment (start 135.73 85.47) (end 135.6 85.6) (width 0.2032) (layer F.Cu) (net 9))
 (segment (start 135.6 85.6) (end 135.6 87.2) (width 0.508) (layer F.Cu) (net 9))
 (segment (start 137.16 88.76) (end 137.16 89.549) (width 0.508) (layer F.Cu) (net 9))
 (segment (start 135.6 87.2) (end 137.16 88.76) (width 0.508) (layer F.Cu) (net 9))
 (segment (start 136.76 85.47) (end 136.76 86.56) (width 0.2032) (layer F.Cu) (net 8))
 (segment (start 136.76 86.56) (end 136.76 87.16) (width 0.508) (layer F.Cu) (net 8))
 (segment (start 138.684 89.084) (end 138.684 89.549) (width 0.508) (layer F.Cu) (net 8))
 (segment (start 136.76 87.16) (end 138.684 89.084) (width 0.508) (layer F.Cu) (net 8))
 (segment (start 137.16 86.241566) (end 138.518434 87.6) (width 0.2032) (layer F.Cu) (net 6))
 (segment (start 137.16 85.47) (end 137.16 86.241566) (width 0.2032) (layer F.Cu) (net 6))
 (segment (start 143.764 88.364) (end 143.764 89.549) (width 0.508) (layer F.Cu) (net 6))
 (segment (start 138.518434 87.6) (end 143 87.6) (width 0.508) (layer F.Cu) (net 6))
 (segment (start 143 87.6) (end 143.764 88.364) (width 0.508) (layer F.Cu) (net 6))
 (segment (start 137.56 86.124936) (end 138.035064 86.6) (width 0.2032) (layer F.Cu) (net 4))
 (segment (start 137.56 85.47) (end 137.56 86.124936) (width 0.2032) (layer F.Cu) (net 4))
 (segment (start 138.035064 86.6) (end 138.4 86.6) (width 0.2032) (layer F.Cu) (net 4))
 (segment (start 145.288 87.688) (end 145.288 89.549) (width 0.508) (layer F.Cu) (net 4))
 (segment (start 144.2 86.6) (end 145.288 87.688) (width 0.508) (layer F.Cu) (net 4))
 (segment (start 138.4 86.6) (end 144.2 86.6) (width 0.508) (layer F.Cu) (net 4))
 (segment (start 137.96 85.47) (end 139.07 85.47) (width 0.2032) (layer F.Cu) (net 2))
 (segment (start 139.07 85.47) (end 145.27 85.47) (width 0.508) (layer F.Cu) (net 2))
 (segment (start 146.812 87.012) (end 146.812 89.549) (width 0.508) (layer F.Cu) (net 2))
 (segment (start 145.27 85.47) (end 146.812 87.012) (width 0.508) (layer F.Cu) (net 2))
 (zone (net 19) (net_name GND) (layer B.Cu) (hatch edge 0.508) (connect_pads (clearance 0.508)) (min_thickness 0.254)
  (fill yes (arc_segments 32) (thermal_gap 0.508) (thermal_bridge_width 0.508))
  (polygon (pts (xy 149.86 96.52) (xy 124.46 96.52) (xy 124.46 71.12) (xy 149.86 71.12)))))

